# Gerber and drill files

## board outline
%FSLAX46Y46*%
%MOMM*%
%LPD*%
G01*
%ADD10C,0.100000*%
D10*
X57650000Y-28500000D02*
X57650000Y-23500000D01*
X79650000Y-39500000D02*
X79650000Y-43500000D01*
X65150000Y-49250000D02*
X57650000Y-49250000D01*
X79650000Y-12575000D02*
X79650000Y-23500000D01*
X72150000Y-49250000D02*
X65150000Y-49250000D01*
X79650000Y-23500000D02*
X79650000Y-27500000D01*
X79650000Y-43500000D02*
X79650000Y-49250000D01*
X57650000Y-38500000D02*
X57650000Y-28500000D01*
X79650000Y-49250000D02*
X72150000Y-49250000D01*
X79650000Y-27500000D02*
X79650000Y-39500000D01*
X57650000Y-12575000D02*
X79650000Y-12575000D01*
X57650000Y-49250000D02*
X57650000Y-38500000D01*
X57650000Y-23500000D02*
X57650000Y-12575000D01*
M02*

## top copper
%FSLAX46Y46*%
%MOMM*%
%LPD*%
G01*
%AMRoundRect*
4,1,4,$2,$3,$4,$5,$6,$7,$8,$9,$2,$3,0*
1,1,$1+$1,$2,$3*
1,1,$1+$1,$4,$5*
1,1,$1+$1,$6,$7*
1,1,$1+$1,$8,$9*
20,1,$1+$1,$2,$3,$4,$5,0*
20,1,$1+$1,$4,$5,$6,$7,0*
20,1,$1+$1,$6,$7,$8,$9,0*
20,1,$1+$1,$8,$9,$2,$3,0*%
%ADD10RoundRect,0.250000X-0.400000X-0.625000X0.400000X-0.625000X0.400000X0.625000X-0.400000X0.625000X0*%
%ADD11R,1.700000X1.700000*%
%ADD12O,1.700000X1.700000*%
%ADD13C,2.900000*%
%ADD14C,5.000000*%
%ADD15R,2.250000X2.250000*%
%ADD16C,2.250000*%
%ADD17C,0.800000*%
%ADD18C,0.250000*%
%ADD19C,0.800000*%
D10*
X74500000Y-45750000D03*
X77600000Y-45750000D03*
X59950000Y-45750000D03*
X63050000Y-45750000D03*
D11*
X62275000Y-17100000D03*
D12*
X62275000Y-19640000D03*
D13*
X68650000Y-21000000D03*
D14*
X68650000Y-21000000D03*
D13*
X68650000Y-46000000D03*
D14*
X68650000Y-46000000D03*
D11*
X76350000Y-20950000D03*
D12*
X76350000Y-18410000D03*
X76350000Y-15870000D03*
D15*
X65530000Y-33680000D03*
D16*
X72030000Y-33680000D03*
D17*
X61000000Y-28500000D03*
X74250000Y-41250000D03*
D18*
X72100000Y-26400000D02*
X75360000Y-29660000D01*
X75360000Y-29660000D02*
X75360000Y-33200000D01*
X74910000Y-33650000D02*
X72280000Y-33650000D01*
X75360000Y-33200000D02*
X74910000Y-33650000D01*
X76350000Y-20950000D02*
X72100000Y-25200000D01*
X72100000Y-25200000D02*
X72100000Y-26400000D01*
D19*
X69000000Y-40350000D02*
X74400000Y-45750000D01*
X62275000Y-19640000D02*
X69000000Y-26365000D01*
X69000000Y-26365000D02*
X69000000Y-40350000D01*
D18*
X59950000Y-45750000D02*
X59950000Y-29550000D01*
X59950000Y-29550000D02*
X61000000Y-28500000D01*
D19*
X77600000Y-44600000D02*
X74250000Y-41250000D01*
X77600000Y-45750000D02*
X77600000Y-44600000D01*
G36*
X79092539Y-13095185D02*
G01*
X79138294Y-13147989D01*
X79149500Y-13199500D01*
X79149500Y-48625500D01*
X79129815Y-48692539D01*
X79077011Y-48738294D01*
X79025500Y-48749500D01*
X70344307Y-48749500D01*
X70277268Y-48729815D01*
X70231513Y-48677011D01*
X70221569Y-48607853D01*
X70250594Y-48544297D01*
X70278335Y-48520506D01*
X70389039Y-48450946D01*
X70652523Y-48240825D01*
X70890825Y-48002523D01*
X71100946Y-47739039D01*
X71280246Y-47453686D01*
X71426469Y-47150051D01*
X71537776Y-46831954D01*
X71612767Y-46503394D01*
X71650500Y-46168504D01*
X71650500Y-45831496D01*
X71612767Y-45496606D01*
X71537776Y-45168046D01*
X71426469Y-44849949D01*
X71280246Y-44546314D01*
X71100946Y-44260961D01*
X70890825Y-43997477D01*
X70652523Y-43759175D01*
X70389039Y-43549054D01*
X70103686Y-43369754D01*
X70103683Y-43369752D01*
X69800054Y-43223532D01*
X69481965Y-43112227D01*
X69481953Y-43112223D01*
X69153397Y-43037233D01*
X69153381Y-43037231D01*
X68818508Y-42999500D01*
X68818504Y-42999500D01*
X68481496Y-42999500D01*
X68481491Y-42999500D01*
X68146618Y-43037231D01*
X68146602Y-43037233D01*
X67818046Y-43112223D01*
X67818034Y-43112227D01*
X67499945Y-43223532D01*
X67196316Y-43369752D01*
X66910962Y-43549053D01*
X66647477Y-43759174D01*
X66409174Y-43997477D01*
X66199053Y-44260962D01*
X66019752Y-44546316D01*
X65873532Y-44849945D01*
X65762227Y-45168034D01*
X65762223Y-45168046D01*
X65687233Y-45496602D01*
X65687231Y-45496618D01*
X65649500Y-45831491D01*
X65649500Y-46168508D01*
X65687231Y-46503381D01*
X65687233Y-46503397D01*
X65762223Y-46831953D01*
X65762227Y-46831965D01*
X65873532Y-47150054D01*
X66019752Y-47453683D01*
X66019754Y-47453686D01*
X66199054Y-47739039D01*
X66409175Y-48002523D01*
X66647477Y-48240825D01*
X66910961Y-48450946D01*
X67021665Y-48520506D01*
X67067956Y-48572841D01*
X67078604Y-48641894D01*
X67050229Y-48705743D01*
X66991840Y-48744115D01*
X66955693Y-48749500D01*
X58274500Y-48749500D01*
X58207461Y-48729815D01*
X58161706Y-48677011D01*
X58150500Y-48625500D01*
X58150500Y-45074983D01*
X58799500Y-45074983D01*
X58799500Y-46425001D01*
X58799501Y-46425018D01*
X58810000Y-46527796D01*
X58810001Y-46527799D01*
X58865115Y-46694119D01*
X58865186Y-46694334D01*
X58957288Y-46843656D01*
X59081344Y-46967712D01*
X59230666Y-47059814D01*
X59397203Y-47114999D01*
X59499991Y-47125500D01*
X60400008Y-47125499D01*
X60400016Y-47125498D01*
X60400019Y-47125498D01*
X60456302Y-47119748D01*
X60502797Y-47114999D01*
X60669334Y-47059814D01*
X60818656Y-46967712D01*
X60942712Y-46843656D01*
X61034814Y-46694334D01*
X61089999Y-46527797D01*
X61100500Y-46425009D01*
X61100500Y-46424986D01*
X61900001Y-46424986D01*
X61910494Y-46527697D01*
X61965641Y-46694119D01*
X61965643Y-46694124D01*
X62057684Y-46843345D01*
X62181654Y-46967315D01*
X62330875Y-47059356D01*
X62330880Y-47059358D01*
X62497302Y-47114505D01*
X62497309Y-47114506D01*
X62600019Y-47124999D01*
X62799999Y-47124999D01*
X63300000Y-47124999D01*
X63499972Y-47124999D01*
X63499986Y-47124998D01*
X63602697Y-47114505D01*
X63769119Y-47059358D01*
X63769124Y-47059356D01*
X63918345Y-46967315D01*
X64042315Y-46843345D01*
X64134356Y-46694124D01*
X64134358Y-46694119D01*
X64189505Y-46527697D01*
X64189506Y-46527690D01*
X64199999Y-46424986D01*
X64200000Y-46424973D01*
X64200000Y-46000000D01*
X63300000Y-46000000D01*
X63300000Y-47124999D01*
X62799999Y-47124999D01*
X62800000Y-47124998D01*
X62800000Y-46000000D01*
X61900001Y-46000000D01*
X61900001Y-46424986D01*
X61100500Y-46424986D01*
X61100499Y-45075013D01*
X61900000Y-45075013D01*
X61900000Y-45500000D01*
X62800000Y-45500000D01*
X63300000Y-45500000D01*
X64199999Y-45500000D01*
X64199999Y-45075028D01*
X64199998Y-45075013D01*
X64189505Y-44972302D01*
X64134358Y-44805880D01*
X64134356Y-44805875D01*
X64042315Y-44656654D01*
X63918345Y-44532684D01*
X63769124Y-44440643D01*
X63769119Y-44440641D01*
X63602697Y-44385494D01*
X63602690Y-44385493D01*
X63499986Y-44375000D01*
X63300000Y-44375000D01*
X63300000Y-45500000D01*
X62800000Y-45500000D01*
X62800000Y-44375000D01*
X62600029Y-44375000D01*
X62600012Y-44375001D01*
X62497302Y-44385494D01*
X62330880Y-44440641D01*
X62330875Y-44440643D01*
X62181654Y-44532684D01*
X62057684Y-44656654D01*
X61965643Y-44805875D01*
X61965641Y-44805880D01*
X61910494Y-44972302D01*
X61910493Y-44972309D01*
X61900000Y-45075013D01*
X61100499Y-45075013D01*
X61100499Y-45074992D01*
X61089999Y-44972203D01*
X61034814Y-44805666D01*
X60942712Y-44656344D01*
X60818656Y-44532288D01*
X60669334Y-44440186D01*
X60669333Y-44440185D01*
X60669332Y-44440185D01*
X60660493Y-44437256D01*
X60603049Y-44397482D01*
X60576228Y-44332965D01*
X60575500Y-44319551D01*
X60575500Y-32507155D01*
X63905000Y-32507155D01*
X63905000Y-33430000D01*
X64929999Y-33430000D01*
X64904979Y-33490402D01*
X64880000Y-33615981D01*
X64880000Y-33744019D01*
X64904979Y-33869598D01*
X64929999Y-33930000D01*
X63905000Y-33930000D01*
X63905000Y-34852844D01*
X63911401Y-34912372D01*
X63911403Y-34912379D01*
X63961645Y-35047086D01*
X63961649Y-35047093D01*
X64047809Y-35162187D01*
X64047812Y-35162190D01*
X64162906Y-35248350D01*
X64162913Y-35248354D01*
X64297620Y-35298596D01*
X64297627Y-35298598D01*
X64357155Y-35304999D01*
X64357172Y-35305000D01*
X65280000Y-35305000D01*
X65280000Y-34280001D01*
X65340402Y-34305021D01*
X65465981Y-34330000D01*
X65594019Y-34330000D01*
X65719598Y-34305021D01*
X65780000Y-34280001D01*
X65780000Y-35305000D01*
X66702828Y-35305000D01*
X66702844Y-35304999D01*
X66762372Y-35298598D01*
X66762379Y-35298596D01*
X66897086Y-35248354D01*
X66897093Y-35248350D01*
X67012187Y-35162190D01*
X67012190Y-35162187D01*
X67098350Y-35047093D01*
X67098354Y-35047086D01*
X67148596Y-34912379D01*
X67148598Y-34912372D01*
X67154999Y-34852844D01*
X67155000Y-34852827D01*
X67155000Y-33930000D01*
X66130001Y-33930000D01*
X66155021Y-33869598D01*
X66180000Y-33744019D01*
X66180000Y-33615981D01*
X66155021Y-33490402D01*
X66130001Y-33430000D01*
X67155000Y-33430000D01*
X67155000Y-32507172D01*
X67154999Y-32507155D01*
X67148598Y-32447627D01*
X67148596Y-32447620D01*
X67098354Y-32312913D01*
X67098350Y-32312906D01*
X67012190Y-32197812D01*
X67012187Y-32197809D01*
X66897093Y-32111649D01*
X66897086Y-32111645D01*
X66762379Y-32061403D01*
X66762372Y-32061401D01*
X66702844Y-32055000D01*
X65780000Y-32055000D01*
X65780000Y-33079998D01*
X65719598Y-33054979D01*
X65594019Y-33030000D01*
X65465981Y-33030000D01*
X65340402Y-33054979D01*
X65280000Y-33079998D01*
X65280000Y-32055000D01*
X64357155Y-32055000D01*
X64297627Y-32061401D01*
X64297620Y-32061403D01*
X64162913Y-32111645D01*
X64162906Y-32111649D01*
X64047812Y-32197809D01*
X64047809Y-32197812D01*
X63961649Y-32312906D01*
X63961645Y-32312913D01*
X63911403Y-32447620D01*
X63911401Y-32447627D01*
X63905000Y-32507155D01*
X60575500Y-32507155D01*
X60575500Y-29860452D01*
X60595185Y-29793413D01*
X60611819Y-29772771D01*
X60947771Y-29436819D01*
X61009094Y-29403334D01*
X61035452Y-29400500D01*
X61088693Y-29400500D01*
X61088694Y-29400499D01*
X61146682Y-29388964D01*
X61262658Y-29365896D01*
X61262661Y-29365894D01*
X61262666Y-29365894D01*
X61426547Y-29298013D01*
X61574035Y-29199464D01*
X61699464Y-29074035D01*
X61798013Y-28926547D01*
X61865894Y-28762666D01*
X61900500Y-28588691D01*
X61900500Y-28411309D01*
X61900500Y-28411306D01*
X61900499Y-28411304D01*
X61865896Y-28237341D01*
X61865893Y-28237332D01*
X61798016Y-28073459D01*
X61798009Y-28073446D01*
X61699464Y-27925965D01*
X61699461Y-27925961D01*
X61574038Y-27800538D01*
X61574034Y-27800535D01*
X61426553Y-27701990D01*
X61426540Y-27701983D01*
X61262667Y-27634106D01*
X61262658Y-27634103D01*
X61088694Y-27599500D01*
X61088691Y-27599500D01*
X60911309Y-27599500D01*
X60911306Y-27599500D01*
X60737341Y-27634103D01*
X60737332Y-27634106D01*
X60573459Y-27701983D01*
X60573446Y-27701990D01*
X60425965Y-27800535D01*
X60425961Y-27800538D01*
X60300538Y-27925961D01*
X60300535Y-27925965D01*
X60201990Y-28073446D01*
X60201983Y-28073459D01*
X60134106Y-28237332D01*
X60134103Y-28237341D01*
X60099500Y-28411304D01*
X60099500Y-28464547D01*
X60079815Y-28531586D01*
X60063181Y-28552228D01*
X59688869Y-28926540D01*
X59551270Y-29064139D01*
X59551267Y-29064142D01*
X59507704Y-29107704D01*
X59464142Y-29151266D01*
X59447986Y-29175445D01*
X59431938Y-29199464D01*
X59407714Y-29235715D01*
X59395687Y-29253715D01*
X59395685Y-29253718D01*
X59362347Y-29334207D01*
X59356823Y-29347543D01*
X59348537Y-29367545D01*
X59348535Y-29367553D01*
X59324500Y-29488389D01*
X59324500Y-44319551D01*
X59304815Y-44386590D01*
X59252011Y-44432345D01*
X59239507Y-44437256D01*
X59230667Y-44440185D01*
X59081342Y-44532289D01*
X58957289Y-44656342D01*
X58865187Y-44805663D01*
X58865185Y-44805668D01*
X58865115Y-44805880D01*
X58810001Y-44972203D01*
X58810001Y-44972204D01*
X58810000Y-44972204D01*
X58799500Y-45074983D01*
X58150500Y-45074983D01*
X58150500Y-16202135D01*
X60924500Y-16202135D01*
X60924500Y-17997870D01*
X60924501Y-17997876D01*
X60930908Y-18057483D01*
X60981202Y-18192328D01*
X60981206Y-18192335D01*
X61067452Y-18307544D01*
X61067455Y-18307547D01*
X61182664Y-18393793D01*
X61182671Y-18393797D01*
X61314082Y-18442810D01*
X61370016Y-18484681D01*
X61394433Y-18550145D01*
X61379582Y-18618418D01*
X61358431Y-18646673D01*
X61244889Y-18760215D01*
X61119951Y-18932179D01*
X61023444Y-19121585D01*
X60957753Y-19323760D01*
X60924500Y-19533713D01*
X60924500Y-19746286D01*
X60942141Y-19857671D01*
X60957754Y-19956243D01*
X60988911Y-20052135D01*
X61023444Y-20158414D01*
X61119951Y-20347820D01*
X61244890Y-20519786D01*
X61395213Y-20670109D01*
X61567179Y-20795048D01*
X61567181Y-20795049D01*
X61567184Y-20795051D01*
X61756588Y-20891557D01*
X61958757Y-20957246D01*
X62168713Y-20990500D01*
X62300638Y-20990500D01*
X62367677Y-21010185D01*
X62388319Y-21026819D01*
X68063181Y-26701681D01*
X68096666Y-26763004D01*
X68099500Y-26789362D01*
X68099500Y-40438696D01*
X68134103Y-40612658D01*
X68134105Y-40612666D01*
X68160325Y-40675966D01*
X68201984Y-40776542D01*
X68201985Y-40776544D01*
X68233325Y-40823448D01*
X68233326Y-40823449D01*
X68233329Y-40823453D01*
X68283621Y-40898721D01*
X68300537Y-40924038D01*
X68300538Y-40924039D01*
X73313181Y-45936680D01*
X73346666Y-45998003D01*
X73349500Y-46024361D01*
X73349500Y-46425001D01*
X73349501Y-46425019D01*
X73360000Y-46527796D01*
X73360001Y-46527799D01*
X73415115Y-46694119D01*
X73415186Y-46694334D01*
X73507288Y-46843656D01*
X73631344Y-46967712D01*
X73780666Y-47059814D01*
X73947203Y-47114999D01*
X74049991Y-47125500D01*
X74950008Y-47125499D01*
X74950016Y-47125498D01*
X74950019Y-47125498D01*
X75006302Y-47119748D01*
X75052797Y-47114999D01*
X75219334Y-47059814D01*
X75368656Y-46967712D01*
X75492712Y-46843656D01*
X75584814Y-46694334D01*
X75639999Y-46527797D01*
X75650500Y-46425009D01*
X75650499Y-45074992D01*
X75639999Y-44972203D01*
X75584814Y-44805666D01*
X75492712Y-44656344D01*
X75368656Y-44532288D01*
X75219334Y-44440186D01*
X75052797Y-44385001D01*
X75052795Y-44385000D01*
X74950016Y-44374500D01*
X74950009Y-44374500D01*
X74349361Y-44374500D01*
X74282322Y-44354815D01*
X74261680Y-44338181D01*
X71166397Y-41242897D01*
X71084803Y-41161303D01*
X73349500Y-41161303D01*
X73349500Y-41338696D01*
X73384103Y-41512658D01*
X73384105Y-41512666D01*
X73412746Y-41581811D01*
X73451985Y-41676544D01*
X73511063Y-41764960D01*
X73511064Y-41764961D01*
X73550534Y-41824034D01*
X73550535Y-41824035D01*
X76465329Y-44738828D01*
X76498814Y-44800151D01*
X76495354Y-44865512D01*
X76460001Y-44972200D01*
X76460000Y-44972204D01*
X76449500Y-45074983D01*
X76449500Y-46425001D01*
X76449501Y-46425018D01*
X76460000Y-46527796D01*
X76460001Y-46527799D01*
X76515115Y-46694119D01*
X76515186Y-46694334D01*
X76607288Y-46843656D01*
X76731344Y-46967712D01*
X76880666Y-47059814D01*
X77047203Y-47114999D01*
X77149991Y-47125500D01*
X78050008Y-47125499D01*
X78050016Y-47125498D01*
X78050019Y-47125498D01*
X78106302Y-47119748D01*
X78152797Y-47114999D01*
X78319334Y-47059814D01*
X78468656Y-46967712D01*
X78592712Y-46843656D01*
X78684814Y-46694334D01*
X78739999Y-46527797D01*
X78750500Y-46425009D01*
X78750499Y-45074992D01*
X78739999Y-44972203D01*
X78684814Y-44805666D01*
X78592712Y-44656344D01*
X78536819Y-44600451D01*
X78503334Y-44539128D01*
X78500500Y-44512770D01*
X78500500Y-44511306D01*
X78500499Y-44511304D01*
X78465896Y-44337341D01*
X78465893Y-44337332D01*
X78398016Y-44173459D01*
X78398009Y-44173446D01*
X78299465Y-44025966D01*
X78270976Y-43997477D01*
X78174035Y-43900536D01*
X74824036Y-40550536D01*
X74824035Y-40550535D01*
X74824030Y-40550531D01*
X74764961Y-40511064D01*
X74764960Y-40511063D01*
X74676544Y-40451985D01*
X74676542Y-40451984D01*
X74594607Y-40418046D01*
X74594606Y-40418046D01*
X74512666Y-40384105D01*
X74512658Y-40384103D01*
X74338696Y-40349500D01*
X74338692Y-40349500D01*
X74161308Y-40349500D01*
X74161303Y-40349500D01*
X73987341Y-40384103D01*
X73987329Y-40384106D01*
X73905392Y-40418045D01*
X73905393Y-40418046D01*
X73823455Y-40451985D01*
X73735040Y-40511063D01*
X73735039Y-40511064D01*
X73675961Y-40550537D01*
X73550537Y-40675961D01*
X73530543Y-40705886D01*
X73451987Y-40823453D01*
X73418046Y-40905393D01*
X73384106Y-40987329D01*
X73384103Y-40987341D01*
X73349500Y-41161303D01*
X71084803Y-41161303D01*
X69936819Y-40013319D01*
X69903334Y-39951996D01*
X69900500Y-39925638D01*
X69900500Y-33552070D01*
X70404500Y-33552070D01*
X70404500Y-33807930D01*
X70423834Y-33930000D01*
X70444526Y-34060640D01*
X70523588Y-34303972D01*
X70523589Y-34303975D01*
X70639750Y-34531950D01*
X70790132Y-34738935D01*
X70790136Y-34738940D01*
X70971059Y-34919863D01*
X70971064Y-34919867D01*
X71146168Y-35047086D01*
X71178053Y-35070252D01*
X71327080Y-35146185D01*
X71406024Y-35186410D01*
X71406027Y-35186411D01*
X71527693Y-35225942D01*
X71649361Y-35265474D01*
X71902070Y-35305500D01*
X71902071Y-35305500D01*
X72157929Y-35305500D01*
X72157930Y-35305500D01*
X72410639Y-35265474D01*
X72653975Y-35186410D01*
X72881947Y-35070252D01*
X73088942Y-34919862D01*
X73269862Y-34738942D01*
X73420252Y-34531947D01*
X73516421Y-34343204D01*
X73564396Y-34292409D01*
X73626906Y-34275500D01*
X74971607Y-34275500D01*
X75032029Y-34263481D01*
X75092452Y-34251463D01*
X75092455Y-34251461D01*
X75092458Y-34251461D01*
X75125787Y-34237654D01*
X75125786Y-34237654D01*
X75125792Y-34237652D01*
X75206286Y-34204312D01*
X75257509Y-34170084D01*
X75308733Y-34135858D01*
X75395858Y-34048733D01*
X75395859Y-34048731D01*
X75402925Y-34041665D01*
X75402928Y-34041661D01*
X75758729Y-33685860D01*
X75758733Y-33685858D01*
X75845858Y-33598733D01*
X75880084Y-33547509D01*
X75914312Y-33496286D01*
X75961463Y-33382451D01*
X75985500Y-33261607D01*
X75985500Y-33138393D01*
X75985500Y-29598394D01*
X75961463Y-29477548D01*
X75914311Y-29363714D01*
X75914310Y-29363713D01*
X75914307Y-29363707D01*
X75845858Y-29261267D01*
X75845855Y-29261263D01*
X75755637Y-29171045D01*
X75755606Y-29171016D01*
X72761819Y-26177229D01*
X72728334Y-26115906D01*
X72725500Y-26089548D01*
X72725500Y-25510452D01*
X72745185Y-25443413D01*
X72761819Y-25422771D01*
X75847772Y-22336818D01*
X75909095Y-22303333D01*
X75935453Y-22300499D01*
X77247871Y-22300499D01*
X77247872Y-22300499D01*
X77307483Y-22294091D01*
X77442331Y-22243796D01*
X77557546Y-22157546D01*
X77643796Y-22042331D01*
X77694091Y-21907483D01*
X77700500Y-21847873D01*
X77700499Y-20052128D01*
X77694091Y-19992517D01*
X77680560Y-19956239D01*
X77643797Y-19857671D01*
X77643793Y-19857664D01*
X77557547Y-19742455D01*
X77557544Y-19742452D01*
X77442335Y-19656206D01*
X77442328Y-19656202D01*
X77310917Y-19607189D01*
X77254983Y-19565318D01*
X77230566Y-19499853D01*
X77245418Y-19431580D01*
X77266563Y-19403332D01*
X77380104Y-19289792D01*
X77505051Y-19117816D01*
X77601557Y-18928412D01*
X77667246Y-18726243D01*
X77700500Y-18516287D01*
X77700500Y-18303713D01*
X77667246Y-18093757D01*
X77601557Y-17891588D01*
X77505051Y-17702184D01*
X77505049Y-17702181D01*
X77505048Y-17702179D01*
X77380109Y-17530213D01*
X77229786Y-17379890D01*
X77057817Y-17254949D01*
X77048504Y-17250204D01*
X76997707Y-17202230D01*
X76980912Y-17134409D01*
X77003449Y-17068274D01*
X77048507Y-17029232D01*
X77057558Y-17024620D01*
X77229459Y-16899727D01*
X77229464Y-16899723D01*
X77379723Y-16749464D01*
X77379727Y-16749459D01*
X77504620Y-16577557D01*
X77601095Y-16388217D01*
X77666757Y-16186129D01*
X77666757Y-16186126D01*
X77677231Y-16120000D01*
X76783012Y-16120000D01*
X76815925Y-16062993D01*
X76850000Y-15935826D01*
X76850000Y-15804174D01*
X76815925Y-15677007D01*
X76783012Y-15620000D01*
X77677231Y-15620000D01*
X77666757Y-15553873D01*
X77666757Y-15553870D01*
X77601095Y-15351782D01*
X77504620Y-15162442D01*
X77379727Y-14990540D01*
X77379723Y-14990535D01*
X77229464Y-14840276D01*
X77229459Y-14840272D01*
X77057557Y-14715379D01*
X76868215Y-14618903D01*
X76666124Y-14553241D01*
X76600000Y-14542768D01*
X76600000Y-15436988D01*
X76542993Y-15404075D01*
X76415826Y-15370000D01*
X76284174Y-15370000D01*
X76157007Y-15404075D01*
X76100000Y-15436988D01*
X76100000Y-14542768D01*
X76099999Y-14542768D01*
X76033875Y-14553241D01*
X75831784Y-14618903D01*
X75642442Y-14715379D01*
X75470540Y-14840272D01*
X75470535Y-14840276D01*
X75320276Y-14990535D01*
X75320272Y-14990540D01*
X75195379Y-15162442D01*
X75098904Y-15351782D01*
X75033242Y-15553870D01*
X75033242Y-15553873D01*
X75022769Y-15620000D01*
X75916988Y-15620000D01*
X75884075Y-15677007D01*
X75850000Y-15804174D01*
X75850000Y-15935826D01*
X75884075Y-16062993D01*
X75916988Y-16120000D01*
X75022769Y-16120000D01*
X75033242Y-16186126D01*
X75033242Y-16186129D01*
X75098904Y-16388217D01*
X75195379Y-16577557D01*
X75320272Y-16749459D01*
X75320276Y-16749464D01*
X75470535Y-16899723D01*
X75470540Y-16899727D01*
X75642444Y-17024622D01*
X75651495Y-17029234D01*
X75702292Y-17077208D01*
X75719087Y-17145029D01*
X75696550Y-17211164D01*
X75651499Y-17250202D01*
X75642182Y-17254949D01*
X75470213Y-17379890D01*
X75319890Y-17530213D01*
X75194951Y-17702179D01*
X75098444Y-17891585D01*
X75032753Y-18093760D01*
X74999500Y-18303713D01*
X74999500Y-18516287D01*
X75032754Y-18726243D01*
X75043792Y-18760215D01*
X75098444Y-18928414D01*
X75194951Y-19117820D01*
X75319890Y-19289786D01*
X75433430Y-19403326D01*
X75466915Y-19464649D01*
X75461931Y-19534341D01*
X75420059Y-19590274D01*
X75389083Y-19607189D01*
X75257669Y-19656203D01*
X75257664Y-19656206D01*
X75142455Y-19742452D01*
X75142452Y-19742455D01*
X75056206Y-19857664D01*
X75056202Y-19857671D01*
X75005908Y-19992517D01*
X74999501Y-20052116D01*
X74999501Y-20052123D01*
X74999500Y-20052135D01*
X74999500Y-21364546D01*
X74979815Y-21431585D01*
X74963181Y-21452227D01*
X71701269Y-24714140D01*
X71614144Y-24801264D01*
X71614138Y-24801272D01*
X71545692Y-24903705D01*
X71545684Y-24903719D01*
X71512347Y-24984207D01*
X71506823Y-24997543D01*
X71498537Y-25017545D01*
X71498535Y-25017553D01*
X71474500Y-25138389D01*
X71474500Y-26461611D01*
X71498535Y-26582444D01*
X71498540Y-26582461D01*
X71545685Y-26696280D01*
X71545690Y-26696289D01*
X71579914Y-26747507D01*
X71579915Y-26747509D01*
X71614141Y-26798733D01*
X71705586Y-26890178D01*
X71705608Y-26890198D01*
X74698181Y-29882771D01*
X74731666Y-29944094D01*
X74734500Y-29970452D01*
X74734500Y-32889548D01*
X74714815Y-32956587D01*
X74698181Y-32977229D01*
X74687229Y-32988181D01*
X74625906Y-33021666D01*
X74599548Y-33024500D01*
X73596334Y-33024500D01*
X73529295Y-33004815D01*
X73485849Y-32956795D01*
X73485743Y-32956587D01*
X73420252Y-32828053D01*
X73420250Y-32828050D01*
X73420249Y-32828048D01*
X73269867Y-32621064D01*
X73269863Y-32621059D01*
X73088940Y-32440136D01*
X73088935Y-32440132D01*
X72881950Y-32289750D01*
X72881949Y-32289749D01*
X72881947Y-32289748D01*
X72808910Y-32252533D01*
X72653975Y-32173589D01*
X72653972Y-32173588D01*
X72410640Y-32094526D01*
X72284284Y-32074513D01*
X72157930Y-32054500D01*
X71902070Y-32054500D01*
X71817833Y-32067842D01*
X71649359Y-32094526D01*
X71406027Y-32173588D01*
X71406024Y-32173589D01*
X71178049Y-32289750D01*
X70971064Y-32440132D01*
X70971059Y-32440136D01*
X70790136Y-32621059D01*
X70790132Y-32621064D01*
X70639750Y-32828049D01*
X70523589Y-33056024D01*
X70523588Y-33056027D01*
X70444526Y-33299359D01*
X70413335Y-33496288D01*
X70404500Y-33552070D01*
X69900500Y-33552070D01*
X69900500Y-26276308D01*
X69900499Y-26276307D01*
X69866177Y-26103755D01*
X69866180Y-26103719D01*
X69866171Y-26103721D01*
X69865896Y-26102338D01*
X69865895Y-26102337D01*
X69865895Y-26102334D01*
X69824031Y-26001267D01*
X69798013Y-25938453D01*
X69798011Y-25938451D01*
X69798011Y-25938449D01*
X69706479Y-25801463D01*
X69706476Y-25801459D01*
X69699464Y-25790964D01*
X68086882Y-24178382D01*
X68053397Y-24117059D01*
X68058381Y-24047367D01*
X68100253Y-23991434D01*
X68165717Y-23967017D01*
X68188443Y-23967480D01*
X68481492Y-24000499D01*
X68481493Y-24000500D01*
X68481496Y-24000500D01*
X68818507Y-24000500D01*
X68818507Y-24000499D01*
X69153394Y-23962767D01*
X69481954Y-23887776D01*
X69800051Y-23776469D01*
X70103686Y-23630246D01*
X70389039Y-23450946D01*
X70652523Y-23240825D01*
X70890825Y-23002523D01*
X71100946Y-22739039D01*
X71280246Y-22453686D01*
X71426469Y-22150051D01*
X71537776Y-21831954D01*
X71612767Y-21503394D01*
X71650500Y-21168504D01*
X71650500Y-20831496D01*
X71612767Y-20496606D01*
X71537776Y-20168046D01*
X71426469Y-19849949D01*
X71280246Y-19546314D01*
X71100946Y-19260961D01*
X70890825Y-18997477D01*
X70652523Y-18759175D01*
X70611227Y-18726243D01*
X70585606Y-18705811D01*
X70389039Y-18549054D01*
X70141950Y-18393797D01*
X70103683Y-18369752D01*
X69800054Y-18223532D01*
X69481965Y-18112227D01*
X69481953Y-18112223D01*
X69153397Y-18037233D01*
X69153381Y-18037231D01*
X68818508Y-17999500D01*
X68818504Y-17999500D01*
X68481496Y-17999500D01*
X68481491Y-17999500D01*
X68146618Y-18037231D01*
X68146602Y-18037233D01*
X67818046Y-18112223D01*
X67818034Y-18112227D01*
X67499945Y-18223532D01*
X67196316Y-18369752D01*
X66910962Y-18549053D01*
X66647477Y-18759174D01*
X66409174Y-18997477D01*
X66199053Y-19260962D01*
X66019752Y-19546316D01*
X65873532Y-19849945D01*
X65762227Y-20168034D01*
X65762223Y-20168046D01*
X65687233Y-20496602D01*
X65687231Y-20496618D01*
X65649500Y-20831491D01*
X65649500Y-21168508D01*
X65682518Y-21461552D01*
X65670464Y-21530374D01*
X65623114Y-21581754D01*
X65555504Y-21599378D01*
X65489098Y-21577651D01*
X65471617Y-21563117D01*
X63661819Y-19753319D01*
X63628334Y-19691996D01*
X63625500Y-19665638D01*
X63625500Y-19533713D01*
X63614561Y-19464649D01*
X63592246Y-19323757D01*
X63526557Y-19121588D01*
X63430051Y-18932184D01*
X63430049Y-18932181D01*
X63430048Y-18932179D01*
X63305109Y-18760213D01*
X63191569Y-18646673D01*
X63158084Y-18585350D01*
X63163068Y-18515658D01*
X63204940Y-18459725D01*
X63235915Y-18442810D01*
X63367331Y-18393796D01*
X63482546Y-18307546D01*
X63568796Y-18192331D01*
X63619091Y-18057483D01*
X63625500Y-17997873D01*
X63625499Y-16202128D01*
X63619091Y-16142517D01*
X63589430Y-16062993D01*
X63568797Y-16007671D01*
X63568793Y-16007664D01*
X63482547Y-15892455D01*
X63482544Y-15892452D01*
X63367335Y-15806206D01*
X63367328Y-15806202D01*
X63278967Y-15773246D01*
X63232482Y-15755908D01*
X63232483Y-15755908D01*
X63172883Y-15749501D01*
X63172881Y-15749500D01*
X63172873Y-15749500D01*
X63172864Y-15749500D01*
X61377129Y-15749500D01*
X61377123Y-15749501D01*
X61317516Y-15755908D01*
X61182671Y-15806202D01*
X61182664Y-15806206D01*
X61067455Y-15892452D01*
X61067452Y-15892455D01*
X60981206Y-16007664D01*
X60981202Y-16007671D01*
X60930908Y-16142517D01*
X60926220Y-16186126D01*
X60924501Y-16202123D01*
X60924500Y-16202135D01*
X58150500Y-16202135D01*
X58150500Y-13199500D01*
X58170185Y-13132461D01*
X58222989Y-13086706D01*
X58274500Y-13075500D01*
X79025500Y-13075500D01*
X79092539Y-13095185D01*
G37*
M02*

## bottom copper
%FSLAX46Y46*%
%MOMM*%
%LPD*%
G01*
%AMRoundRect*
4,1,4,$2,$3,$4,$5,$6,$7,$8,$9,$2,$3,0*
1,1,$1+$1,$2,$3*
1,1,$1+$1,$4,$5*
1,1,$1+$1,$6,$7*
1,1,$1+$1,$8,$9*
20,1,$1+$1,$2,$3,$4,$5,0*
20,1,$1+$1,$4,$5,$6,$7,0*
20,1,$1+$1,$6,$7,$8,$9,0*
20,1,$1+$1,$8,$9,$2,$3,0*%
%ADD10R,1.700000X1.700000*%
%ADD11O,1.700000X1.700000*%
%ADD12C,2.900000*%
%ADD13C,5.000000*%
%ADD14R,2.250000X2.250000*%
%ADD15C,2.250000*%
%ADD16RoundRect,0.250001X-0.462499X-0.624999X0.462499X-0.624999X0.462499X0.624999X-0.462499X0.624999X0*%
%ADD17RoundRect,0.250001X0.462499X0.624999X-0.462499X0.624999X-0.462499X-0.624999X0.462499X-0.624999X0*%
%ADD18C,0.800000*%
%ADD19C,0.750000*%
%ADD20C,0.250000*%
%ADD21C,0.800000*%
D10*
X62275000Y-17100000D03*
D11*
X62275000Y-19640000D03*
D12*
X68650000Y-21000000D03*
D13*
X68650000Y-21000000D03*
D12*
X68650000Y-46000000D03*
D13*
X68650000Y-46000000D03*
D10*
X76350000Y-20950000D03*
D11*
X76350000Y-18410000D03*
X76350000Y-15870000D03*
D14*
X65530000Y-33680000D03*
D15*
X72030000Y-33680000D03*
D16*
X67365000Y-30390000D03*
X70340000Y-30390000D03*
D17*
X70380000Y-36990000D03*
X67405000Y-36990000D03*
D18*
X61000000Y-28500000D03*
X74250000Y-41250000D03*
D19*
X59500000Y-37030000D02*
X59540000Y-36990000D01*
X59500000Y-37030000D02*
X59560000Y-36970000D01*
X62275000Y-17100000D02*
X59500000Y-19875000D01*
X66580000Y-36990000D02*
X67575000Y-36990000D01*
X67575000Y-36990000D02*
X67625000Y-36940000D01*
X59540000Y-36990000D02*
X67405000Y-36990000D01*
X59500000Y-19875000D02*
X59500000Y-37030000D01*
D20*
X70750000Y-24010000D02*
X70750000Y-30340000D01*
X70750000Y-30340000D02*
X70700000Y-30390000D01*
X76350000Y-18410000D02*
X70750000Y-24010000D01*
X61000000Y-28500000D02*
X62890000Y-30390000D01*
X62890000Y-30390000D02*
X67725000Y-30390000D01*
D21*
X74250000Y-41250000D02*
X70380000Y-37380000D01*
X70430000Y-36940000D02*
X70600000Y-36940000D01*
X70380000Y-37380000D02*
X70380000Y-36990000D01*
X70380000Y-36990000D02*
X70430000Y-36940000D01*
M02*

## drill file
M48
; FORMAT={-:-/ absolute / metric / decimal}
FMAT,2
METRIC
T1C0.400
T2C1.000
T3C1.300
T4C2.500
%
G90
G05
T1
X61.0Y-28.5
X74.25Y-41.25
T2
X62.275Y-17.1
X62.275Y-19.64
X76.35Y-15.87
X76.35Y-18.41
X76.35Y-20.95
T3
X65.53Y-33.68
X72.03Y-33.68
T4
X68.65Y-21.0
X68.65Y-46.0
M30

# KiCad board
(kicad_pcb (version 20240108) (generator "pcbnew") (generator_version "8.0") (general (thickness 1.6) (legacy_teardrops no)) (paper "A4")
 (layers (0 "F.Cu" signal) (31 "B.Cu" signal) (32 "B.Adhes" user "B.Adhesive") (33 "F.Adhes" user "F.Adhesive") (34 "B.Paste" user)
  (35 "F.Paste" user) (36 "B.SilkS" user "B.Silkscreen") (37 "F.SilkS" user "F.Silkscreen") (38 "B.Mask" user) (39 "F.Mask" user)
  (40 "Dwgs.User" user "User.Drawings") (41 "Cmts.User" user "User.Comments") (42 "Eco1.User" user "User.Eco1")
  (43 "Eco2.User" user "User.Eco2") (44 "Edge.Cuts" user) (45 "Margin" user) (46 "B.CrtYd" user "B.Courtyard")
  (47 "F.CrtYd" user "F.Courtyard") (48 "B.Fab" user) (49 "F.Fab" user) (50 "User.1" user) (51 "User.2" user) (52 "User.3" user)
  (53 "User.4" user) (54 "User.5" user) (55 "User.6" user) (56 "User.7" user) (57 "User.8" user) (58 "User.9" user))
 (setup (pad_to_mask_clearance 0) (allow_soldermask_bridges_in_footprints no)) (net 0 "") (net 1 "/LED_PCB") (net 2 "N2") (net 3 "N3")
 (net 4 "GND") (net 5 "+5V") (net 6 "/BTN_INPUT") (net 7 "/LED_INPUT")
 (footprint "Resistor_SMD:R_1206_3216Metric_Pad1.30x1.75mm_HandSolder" (layer "F.Cu") (at 76.05 45.75)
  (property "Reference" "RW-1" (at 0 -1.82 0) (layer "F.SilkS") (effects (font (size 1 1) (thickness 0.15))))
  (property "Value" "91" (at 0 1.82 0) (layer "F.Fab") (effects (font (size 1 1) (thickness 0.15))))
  (pad "1" smd roundrect (at -1.55 0) (size 1.3 1.75) (layers "F.Cu" "F.Paste" "F.Mask") (roundrect_rratio 0.192308) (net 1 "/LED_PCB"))
  (pad "2" smd roundrect (at 1.55 0) (size 1.3 1.75) (layers "F.Cu" "F.Paste" "F.Mask") (roundrect_rratio 0.192308) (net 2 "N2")))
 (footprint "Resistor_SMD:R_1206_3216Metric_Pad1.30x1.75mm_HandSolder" (layer "F.Cu") (at 61.5 45.75)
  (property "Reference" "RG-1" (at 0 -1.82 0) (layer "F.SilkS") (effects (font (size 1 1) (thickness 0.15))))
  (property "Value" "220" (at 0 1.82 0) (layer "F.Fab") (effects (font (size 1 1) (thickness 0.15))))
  (pad "1" smd roundrect (at -1.55 0) (size 1.3 1.75) (layers "F.Cu" "F.Paste" "F.Mask") (roundrect_rratio 0.192308) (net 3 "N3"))
  (pad "2" smd roundrect (at 1.55 0) (size 1.3 1.75) (layers "F.Cu" "F.Paste" "F.Mask") (roundrect_rratio 0.192308) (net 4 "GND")))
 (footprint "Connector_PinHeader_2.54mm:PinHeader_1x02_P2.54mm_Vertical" (layer "F.Cu") (at 62.275 17.1)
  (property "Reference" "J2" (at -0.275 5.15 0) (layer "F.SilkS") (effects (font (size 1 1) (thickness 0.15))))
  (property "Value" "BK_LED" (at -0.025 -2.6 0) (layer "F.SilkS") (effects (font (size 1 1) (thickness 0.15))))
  (pad "1" thru_hole rect (at 0 0) (size 1.7 1.7) (drill 1) (layers "*.Cu" "*.Mask") (remove_unused_layers no) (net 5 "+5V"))
  (pad "2" thru_hole oval (at 0 2.54) (size 1.7 1.7) (drill 1) (layers "*.Cu" "*.Mask") (remove_unused_layers no) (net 1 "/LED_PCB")))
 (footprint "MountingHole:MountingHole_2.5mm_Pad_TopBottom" (layer "F.Cu") (at 68.65 21 180)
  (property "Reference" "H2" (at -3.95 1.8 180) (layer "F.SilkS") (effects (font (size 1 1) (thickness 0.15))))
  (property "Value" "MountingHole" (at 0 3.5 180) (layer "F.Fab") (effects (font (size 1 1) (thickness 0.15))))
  (pad "1" thru_hole circle (at 0 0 180) (size 2.9 2.9) (drill 2.5) (layers "*.Cu" "*.Mask") (remove_unused_layers no))
  (pad "1" connect circle (at 0 0 180) (size 5 5) (layers "F.Cu" "F.Mask"))
  (pad "1" connect circle (at 0 0 180) (size 5 5) (layers "B.Cu" "B.Mask")))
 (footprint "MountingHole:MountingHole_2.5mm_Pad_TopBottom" (layer "F.Cu") (at 68.65 46 180)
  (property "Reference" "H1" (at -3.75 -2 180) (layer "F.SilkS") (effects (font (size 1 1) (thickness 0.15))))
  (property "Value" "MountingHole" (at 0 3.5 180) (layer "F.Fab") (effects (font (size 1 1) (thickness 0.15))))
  (pad "1" thru_hole circle (at 0 0 180) (size 2.9 2.9) (drill 2.5) (layers "*.Cu" "*.Mask") (remove_unused_layers no))
  (pad "1" connect circle (at 0 0 180) (size 5 5) (layers "F.Cu" "F.Mask"))
  (pad "1" connect circle (at 0 0 180) (size 5 5) (layers "B.Cu" "B.Mask")))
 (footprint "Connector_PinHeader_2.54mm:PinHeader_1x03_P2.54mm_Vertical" (layer "F.Cu") (at 76.35 20.95 180)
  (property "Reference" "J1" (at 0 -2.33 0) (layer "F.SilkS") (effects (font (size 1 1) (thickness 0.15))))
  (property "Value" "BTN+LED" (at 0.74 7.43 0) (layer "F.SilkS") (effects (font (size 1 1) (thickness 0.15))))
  (pad "1" thru_hole rect (at 0 0 180) (size 1.7 1.7) (drill 1) (layers "*.Cu" "*.Mask") (remove_unused_layers no) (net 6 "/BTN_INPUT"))
  (pad "2" thru_hole oval (at 0 2.54 180) (size 1.7 1.7) (drill 1) (layers "*.Cu" "*.Mask") (remove_unused_layers no) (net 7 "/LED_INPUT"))
  (pad "3" thru_hole oval (at 0 5.08 180) (size 1.7 1.7) (drill 1) (layers "*.Cu" "*.Mask") (remove_unused_layers no) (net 4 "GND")))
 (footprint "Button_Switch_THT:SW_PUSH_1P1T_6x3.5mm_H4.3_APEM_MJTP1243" (layer "B.Cu") (at 65.53 33.68)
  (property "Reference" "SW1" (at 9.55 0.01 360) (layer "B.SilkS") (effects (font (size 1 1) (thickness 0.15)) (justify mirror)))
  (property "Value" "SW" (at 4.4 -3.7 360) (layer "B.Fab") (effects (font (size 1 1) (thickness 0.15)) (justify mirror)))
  (pad "1" thru_hole rect (at 0 0 270) (size 2.25 2.25) (drill 1.3) (layers "*.Cu" "*.Mask") (remove_unused_layers no) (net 4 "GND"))
  (pad "2" thru_hole circle (at 6.5 0 270) (size 2.25 2.25) (drill 1.3) (layers "*.Cu" "*.Mask") (remove_unused_layers no)
   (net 6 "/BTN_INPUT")))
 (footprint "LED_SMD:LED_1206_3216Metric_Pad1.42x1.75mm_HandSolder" (layer "B.Cu") (at 68.8525 30.39)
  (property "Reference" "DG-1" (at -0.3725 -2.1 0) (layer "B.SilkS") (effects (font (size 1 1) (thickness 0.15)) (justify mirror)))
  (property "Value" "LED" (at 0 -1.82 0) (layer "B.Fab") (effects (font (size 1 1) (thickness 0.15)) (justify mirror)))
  (pad "1" smd roundrect (at -1.4875 0) (size 1.425 1.75) (layers "B.Cu" "B.Paste" "B.Mask") (roundrect_rratio 0.175439) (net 3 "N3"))
  (pad "2" smd roundrect (at 1.4875 0) (size 1.425 1.75) (layers "B.Cu" "B.Paste" "B.Mask") (roundrect_rratio 0.175439) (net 7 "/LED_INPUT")))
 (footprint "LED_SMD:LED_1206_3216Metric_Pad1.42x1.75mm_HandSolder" (layer "B.Cu") (at 68.8925 36.99 180)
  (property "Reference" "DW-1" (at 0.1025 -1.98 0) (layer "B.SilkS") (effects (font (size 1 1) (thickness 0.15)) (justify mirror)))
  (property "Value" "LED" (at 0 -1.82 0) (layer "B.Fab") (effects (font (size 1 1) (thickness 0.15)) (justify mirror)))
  (pad "1" smd roundrect (at -1.4875 0 180) (size 1.425 1.75) (layers "B.Cu" "B.Paste" "B.Mask") (roundrect_rratio 0.175439) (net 2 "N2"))
  (pad "2" smd roundrect (at 1.4875 0 180) (size 1.425 1.75) (layers "B.Cu" "B.Paste" "B.Mask") (roundrect_rratio 0.175439) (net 5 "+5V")))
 (gr_line (start 57.65 28.5) (end 57.65 23.5) (stroke (width 0.1) (type default)) (layer "Edge.Cuts"))
 (gr_line (start 79.65 39.5) (end 79.65 43.5) (stroke (width 0.1) (type default)) (layer "Edge.Cuts"))
 (gr_line (start 65.15 49.25) (end 57.65 49.25) (stroke (width 0.1) (type default)) (layer "Edge.Cuts"))
 (gr_line (start 79.65 12.575) (end 79.65 23.5) (stroke (width 0.1) (type default)) (layer "Edge.Cuts"))
 (gr_line (start 72.15 49.25) (end 65.15 49.25) (stroke (width 0.1) (type default)) (layer "Edge.Cuts"))
 (gr_line (start 79.65 23.5) (end 79.65 27.5) (stroke (width 0.1) (type default)) (layer "Edge.Cuts"))
 (gr_line (start 79.65 43.5) (end 79.65 49.25) (stroke (width 0.1) (type default)) (layer "Edge.Cuts"))
 (gr_line (start 57.65 38.5) (end 57.65 28.5) (stroke (width 0.1) (type default)) (layer "Edge.Cuts"))
 (gr_line (start 79.65 49.25) (end 72.15 49.25) (stroke (width 0.1) (type default)) (layer "Edge.Cuts"))
 (gr_line (start 79.65 27.5) (end 79.65 39.5) (stroke (width 0.1) (type default)) (layer "Edge.Cuts"))
 (gr_line (start 57.65 12.575) (end 79.65 12.575) (stroke (width 0.1) (type default)) (layer "Edge.Cuts"))
 (gr_line (start 57.65 49.25) (end 57.65 38.5) (stroke (width 0.1) (type default)) (layer "Edge.Cuts"))
 (gr_line (start 57.65 23.5) (end 57.65 12.575) (stroke (width 0.1) (type default)) (layer "Edge.Cuts"))
 (segment (start 59.5 37.03) (end 59.54 36.99) (width 0.75) (layer "B.Cu") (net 5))
 (segment (start 59.5 37.03) (end 59.56 36.97) (width 0.75) (layer "B.Cu") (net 5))
 (segment (start 62.275 17.1) (end 59.5 19.875) (width 0.75) (layer "B.Cu") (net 5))
 (segment (start 66.58 36.99) (end 67.575 36.99) (width 0.75) (layer "B.Cu") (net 5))
 (segment (start 67.575 36.99) (end 67.625 36.94) (width 0.75) (layer "B.Cu") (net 5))
 (segment (start 59.54 36.99) (end 67.405 36.99) (width 0.75) (layer "B.Cu") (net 5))
 (segment (start 59.5 19.875) (end 59.5 37.03) (width 0.75) (layer "B.Cu") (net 5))
 (segment (start 70.75 24.01) (end 70.75 30.34) (width 0.25) (layer "B.Cu") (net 7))
 (segment (start 70.75 30.34) (end 70.7 30.39) (width 0.25) (layer "B.Cu") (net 7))
 (segment (start 76.35 18.41) (end 70.75 24.01) (width 0.25) (layer "B.Cu") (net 7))
 (segment (start 72.1 26.4) (end 75.36 29.66) (width 0.25) (layer "F.Cu") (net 6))
 (segment (start 75.36 29.66) (end 75.36 33.2) (width 0.25) (layer "F.Cu") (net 6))
 (segment (start 74.91 33.65) (end 72.28 33.65) (width 0.25) (layer "F.Cu") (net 6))
 (segment (start 75.36 33.2) (end 74.91 33.65) (width 0.25) (layer "F.Cu") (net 6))
 (segment (start 76.35 20.95) (end 72.1 25.2) (width 0.25) (layer "F.Cu") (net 6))
 (segment (start 72.1 25.2) (end 72.1 26.4) (width 0.25) (layer "F.Cu") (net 6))
 (segment (start 69 40.35) (end 74.4 45.75) (width 0.8) (layer "F.Cu") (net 1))
 (segment (start 62.275 19.64) (end 69 26.365) (width 0.8) (layer "F.Cu") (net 1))
 (segment (start 69 26.365) (end 69 40.35) (width 0.8) (layer "F.Cu") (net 1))
 (segment (start 59.95 45.75) (end 59.95 29.55) (width 0.25) (layer "F.Cu") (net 3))
 (segment (start 59.95 29.55) (end 61 28.5) (width 0.25) (layer "F.Cu") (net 3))
 (via (at 61 28.5) (size 0.8) (drill 0.4) (layers "F.Cu" "B.Cu") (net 3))
 (segment (start 61 28.5) (end 62.89 30.39) (width 0.25) (layer "B.Cu") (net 3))
 (segment (start 62.89 30.39) (end 67.725 30.39) (width 0.25) (layer "B.Cu") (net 3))
 (segment (start 77.6 44.6) (end 74.25 41.25) (width 0.8) (layer "F.Cu") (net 2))
 (segment (start 77.6 45.75) (end 77.6 44.6) (width 0.8) (layer "F.Cu") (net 2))
 (via (at 74.25 41.25) (size 0.8) (drill 0.4) (layers "F.Cu" "B.Cu") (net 2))
 (segment (start 74.25 41.25) (end 70.38 37.38) (width 0.8) (layer "B.Cu") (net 2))
 (segment (start 70.43 36.94) (end 70.6 36.94) (width 0.8) (layer "B.Cu") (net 2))
 (segment (start 70.38 37.38) (end 70.38 36.99) (width 0.8) (layer "B.Cu") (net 2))
 (segment (start 70.38 36.99) (end 70.43 36.94) (width 0.8) (layer "B.Cu") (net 2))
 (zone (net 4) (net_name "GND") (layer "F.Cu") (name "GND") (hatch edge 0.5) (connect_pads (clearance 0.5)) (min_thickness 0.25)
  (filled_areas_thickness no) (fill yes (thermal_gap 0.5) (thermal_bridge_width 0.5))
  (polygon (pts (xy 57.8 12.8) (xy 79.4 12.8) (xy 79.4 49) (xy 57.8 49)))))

